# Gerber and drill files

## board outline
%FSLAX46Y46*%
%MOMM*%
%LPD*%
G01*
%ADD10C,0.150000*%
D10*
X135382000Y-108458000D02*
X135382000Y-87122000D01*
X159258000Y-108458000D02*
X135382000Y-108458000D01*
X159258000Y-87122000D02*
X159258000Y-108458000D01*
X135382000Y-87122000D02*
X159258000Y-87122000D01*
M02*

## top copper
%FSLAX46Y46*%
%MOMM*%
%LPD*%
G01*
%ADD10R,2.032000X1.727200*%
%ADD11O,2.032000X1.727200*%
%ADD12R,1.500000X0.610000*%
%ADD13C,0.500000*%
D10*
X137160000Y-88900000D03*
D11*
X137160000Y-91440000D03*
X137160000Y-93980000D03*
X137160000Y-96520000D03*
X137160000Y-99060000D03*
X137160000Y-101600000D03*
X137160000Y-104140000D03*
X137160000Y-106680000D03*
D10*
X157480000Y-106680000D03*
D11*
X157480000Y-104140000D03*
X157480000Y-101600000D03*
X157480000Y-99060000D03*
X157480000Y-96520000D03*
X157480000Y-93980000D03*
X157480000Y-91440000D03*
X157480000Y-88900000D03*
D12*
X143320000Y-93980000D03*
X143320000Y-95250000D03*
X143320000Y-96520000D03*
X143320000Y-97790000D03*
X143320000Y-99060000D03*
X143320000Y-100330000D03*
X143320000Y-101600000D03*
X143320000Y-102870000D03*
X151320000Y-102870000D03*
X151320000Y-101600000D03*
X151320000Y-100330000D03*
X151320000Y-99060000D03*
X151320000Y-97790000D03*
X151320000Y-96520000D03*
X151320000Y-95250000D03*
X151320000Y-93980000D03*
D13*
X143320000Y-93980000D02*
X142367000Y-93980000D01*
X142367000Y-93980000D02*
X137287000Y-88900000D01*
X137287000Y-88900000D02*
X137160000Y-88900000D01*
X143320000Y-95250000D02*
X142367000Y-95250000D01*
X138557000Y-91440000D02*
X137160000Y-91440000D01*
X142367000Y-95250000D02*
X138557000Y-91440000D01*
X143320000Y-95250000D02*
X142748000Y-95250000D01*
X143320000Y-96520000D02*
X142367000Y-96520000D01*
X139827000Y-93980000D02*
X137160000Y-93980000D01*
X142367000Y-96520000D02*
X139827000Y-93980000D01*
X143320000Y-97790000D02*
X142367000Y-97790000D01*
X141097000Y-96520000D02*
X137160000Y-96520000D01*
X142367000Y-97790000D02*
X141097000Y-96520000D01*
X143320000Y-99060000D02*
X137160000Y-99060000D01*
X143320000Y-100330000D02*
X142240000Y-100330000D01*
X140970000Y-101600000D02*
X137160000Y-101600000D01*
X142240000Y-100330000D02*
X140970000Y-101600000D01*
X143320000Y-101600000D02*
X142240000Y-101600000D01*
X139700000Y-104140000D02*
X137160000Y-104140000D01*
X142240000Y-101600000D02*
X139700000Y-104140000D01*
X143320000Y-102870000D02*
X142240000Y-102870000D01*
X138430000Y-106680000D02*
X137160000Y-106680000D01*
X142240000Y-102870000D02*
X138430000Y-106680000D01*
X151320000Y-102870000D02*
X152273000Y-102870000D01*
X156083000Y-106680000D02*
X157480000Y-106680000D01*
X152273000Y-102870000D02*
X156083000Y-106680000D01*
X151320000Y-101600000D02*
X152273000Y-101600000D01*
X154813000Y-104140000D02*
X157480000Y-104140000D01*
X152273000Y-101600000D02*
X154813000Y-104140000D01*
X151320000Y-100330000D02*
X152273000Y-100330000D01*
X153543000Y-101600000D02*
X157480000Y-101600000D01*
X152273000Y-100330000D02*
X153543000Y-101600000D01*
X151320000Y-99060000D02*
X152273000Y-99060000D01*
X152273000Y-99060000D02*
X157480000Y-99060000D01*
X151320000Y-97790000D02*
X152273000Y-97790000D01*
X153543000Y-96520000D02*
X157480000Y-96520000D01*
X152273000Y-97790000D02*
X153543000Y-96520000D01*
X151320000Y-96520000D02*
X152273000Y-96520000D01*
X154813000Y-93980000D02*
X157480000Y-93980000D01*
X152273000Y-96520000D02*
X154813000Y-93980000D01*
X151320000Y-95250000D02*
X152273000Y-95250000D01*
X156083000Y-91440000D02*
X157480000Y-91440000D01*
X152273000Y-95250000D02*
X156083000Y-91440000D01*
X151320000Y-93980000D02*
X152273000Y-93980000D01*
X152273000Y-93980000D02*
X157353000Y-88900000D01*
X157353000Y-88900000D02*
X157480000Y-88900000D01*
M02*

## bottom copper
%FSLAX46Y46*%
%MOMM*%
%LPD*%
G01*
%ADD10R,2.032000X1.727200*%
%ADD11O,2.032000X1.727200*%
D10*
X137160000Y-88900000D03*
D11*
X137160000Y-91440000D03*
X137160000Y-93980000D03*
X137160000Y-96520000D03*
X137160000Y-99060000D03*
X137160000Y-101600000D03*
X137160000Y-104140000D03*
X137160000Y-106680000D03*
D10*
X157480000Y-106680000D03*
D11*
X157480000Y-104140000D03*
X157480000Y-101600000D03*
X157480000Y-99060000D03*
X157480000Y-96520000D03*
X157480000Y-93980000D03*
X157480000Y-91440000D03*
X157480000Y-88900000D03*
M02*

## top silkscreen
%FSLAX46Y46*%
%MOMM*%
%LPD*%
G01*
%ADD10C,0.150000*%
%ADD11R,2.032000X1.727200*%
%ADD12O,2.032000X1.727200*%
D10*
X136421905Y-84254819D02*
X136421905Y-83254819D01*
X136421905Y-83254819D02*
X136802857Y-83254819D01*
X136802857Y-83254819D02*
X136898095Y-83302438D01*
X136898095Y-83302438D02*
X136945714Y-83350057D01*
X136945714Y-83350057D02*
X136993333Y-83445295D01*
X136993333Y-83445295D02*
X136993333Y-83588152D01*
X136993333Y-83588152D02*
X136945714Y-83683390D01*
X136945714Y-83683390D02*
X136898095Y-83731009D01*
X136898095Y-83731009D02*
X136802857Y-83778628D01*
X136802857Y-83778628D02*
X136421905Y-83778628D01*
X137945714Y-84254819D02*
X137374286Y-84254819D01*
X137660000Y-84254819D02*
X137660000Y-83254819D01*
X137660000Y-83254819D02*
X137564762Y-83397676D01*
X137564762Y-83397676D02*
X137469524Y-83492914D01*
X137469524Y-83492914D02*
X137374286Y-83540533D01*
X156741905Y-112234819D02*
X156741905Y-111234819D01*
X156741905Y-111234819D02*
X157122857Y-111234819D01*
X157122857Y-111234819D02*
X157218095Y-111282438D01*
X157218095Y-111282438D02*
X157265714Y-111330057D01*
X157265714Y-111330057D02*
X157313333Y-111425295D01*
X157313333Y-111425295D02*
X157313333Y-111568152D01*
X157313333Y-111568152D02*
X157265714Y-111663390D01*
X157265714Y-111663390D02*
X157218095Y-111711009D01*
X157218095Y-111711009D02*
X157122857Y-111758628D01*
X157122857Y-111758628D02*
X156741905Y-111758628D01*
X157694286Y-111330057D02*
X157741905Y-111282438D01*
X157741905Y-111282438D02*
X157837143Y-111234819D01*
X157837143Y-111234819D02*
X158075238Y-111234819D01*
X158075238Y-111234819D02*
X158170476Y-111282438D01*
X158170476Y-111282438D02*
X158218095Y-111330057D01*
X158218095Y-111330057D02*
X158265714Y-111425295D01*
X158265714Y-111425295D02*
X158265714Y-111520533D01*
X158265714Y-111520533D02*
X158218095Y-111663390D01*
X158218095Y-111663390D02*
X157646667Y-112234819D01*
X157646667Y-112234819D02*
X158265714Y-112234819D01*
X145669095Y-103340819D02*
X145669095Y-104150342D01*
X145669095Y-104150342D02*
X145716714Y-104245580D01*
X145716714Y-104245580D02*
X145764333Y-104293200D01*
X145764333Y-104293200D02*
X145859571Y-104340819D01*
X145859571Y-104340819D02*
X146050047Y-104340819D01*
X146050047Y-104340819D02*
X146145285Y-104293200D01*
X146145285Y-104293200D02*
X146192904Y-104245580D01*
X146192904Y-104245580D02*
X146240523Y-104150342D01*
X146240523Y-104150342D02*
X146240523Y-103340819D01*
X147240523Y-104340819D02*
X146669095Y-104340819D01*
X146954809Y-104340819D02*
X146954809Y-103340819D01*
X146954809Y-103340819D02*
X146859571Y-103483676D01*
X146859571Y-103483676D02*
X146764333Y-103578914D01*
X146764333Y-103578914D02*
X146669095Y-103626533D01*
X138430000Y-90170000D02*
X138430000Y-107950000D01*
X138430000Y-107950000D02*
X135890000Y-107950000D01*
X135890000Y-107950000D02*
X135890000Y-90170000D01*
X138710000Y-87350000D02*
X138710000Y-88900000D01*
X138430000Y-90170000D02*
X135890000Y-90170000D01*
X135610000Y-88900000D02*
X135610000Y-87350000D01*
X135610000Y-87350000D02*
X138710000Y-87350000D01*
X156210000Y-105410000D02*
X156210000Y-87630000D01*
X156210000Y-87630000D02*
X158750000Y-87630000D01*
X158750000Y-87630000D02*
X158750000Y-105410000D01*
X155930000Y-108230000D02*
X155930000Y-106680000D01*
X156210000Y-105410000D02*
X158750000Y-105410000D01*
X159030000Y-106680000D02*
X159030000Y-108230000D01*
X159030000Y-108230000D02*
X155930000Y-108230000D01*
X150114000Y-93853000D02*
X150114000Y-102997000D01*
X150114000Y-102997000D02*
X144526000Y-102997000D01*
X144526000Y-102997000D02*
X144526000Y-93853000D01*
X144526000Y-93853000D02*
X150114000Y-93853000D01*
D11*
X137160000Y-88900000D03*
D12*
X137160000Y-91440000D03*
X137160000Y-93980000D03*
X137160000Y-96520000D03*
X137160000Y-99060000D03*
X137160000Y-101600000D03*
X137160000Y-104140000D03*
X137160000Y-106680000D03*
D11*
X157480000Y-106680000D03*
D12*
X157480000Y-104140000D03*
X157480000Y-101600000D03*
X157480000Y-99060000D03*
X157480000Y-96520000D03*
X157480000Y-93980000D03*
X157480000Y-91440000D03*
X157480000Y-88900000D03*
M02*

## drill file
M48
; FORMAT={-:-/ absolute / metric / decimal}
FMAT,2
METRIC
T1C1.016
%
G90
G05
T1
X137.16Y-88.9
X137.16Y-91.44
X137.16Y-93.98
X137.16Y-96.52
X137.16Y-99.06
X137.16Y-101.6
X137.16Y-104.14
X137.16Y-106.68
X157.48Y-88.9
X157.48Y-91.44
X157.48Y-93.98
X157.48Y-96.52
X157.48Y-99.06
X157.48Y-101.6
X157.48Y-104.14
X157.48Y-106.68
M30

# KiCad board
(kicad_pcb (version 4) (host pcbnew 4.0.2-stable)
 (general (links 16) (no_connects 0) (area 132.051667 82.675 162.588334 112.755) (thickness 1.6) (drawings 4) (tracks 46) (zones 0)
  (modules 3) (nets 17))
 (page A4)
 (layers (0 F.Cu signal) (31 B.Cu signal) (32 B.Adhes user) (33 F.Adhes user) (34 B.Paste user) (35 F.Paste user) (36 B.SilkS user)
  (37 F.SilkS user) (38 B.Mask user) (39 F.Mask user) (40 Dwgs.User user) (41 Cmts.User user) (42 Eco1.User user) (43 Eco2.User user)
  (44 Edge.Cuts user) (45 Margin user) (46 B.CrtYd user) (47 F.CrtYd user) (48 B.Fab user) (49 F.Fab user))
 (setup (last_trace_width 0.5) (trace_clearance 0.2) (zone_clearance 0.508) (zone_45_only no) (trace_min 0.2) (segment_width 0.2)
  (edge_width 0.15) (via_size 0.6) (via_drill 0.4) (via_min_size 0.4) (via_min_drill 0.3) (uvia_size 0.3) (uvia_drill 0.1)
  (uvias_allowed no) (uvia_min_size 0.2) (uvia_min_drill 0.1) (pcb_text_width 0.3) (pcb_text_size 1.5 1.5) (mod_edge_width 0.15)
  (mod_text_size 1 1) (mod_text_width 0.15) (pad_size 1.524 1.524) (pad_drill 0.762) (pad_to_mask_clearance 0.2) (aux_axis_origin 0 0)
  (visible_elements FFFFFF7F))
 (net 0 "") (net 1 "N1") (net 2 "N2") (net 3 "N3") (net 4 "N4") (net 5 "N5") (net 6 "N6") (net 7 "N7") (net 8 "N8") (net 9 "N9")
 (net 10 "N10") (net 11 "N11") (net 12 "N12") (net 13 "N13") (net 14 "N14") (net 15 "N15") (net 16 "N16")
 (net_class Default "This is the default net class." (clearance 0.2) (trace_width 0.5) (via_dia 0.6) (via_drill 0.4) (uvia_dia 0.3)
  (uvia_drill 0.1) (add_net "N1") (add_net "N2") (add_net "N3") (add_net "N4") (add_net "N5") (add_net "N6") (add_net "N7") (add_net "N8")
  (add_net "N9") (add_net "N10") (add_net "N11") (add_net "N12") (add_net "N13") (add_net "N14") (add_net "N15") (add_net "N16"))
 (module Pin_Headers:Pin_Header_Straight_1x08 (layer F.Cu) (at 137.16 88.9)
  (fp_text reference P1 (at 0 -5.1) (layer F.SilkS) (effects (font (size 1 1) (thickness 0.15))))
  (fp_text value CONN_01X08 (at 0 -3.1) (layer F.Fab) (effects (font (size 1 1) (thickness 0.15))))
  (fp_line (start 1.27 1.27) (end 1.27 19.05) (layer F.SilkS) (width 0.15))
  (fp_line (start 1.27 19.05) (end -1.27 19.05) (layer F.SilkS) (width 0.15))
  (fp_line (start -1.27 19.05) (end -1.27 1.27) (layer F.SilkS) (width 0.15))
  (fp_line (start 1.55 -1.55) (end 1.55 0) (layer F.SilkS) (width 0.15))
  (fp_line (start 1.27 1.27) (end -1.27 1.27) (layer F.SilkS) (width 0.15))
  (fp_line (start -1.55 0) (end -1.55 -1.55) (layer F.SilkS) (width 0.15))
  (fp_line (start -1.55 -1.55) (end 1.55 -1.55) (layer F.SilkS) (width 0.15))
  (pad 1 thru_hole rect (at 0 0) (size 2.032 1.7272) (drill 1.016) (layers *.Cu *.Mask F.SilkS) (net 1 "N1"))
  (pad 2 thru_hole oval (at 0 2.54) (size 2.032 1.7272) (drill 1.016) (layers *.Cu *.Mask F.SilkS) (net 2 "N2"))
  (pad 3 thru_hole oval (at 0 5.08) (size 2.032 1.7272) (drill 1.016) (layers *.Cu *.Mask F.SilkS) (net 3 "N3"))
  (pad 4 thru_hole oval (at 0 7.62) (size 2.032 1.7272) (drill 1.016) (layers *.Cu *.Mask F.SilkS) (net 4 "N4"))
  (pad 5 thru_hole oval (at 0 10.16) (size 2.032 1.7272) (drill 1.016) (layers *.Cu *.Mask F.SilkS) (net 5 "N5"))
  (pad 6 thru_hole oval (at 0 12.7) (size 2.032 1.7272) (drill 1.016) (layers *.Cu *.Mask F.SilkS) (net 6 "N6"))
  (pad 7 thru_hole oval (at 0 15.24) (size 2.032 1.7272) (drill 1.016) (layers *.Cu *.Mask F.SilkS) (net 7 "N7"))
  (pad 8 thru_hole oval (at 0 17.78) (size 2.032 1.7272) (drill 1.016) (layers *.Cu *.Mask F.SilkS) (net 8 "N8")))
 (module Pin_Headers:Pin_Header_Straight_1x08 (layer F.Cu) (at 157.48 106.68 180)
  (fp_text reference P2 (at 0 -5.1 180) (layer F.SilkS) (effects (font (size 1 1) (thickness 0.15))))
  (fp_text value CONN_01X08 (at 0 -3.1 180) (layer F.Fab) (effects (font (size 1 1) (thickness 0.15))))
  (fp_line (start 1.27 1.27) (end 1.27 19.05) (layer F.SilkS) (width 0.15))
  (fp_line (start 1.27 19.05) (end -1.27 19.05) (layer F.SilkS) (width 0.15))
  (fp_line (start -1.27 19.05) (end -1.27 1.27) (layer F.SilkS) (width 0.15))
  (fp_line (start 1.55 -1.55) (end 1.55 0) (layer F.SilkS) (width 0.15))
  (fp_line (start 1.27 1.27) (end -1.27 1.27) (layer F.SilkS) (width 0.15))
  (fp_line (start -1.55 0) (end -1.55 -1.55) (layer F.SilkS) (width 0.15))
  (fp_line (start -1.55 -1.55) (end 1.55 -1.55) (layer F.SilkS) (width 0.15))
  (pad 1 thru_hole rect (at 0 0 180) (size 2.032 1.7272) (drill 1.016) (layers *.Cu *.Mask F.SilkS) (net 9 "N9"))
  (pad 2 thru_hole oval (at 0 2.54 180) (size 2.032 1.7272) (drill 1.016) (layers *.Cu *.Mask F.SilkS) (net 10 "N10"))
  (pad 3 thru_hole oval (at 0 5.08 180) (size 2.032 1.7272) (drill 1.016) (layers *.Cu *.Mask F.SilkS) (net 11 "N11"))
  (pad 4 thru_hole oval (at 0 7.62 180) (size 2.032 1.7272) (drill 1.016) (layers *.Cu *.Mask F.SilkS) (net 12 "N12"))
  (pad 5 thru_hole oval (at 0 10.16 180) (size 2.032 1.7272) (drill 1.016) (layers *.Cu *.Mask F.SilkS) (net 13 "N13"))
  (pad 6 thru_hole oval (at 0 12.7 180) (size 2.032 1.7272) (drill 1.016) (layers *.Cu *.Mask F.SilkS) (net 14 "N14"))
  (pad 7 thru_hole oval (at 0 15.24 180) (size 2.032 1.7272) (drill 1.016) (layers *.Cu *.Mask F.SilkS) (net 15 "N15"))
  (pad 8 thru_hole oval (at 0 17.78 180) (size 2.032 1.7272) (drill 1.016) (layers *.Cu *.Mask F.SilkS) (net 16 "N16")))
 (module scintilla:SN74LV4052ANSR (layer F.Cu) (at 147.32 99.06 270)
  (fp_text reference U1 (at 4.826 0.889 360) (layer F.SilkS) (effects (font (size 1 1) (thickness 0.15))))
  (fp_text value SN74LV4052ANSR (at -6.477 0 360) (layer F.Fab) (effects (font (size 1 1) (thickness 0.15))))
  (fp_line (start -5.207 -2.794) (end 3.937 -2.794) (layer F.SilkS) (width 0.15))
  (fp_line (start 3.937 -2.794) (end 3.937 2.794) (layer F.SilkS) (width 0.15))
  (fp_line (start 3.937 2.794) (end -5.207 2.794) (layer F.SilkS) (width 0.15))
  (fp_line (start -5.207 2.794) (end -5.207 -2.794) (layer F.SilkS) (width 0.15))
  (pad 1 smd rect (at -5.08 4 270) (size 0.61 1.5) (layers F.Cu F.Paste F.Mask) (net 1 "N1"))
  (pad 2 smd rect (at -3.81 4 270) (size 0.61 1.5) (layers F.Cu F.Paste F.Mask) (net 2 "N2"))
  (pad 3 smd rect (at -2.54 4 270) (size 0.61 1.5) (layers F.Cu F.Paste F.Mask) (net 3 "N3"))
  (pad 4 smd rect (at -1.27 4 270) (size 0.61 1.5) (layers F.Cu F.Paste F.Mask) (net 4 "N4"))
  (pad 5 smd rect (at 0 4 270) (size 0.61 1.5) (layers F.Cu F.Paste F.Mask) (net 5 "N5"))
  (pad 6 smd rect (at 1.27 4 270) (size 0.61 1.5) (layers F.Cu F.Paste F.Mask) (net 6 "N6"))
  (pad 7 smd rect (at 2.54 4 270) (size 0.61 1.5) (layers F.Cu F.Paste F.Mask) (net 7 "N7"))
  (pad 8 smd rect (at 3.81 4 270) (size 0.61 1.5) (layers F.Cu F.Paste F.Mask) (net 8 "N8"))
  (pad 9 smd rect (at 3.81 -4 270) (size 0.61 1.5) (layers F.Cu F.Paste F.Mask) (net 9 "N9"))
  (pad 10 smd rect (at 2.54 -4 270) (size 0.61 1.5) (layers F.Cu F.Paste F.Mask) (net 10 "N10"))
  (pad 11 smd rect (at 1.27 -4 270) (size 0.61 1.5) (layers F.Cu F.Paste F.Mask) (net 11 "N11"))
  (pad 12 smd rect (at 0 -4 270) (size 0.61 1.5) (layers F.Cu F.Paste F.Mask) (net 12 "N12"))
  (pad 13 smd rect (at -1.27 -4 270) (size 0.61 1.5) (layers F.Cu F.Paste F.Mask) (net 13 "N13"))
  (pad 14 smd rect (at -2.54 -4 270) (size 0.61 1.5) (layers F.Cu F.Paste F.Mask) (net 14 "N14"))
  (pad 15 smd rect (at -3.81 -4 270) (size 0.61 1.5) (layers F.Cu F.Paste F.Mask) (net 15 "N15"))
  (pad 16 smd rect (at -5.08 -4 270) (size 0.61 1.5) (layers F.Cu F.Paste F.Mask) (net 16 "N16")))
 (gr_line (start 135.382 108.458) (end 135.382 87.122) (angle 90) (layer Edge.Cuts) (width 0.15))
 (gr_line (start 159.258 108.458) (end 135.382 108.458) (angle 90) (layer Edge.Cuts) (width 0.15))
 (gr_line (start 159.258 87.122) (end 159.258 108.458) (angle 90) (layer Edge.Cuts) (width 0.15))
 (gr_line (start 135.382 87.122) (end 159.258 87.122) (angle 90) (layer Edge.Cuts) (width 0.15))
 (segment (start 143.32 93.98) (end 142.367 93.98) (width 0.5) (layer F.Cu) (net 1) (status 400000))
 (segment (start 142.367 93.98) (end 137.287 88.9) (width 0.5) (layer F.Cu) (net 1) (status 800000))
 (segment (start 137.287 88.9) (end 137.16 88.9) (width 0.5) (layer F.Cu) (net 1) (status C00000))
 (segment (start 143.32 95.25) (end 142.367 95.25) (width 0.5) (layer F.Cu) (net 2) (status 400000))
 (segment (start 138.557 91.44) (end 137.16 91.44) (width 0.5) (layer F.Cu) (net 2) (status 800000))
 (segment (start 142.367 95.25) (end 138.557 91.44) (width 0.5) (layer F.Cu) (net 2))
 (segment (start 143.32 95.25) (end 142.748 95.25) (width 0.5) (layer F.Cu) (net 2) (status C00000))
 (segment (start 143.32 96.52) (end 142.367 96.52) (width 0.5) (layer F.Cu) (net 3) (status 400000))
 (segment (start 139.827 93.98) (end 137.16 93.98) (width 0.5) (layer F.Cu) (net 3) (status 800000))
 (segment (start 142.367 96.52) (end 139.827 93.98) (width 0.5) (layer F.Cu) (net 3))
 (segment (start 143.32 97.79) (end 142.367 97.79) (width 0.5) (layer F.Cu) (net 4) (status 400000))
 (segment (start 141.097 96.52) (end 137.16 96.52) (width 0.5) (layer F.Cu) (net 4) (status 800000))
 (segment (start 142.367 97.79) (end 141.097 96.52) (width 0.5) (layer F.Cu) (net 4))
 (segment (start 143.32 99.06) (end 137.16 99.06) (width 0.5) (layer F.Cu) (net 5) (status C00000))
 (segment (start 143.32 100.33) (end 142.24 100.33) (width 0.5) (layer F.Cu) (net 6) (status 400000))
 (segment (start 140.97 101.6) (end 137.16 101.6) (width 0.5) (layer F.Cu) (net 6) (status 800000))
 (segment (start 142.24 100.33) (end 140.97 101.6) (width 0.5) (layer F.Cu) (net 6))
 (segment (start 143.32 101.6) (end 142.24 101.6) (width 0.5) (layer F.Cu) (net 7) (status 400000))
 (segment (start 139.7 104.14) (end 137.16 104.14) (width 0.5) (layer F.Cu) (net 7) (status 800000))
 (segment (start 142.24 101.6) (end 139.7 104.14) (width 0.5) (layer F.Cu) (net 7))
 (segment (start 143.32 102.87) (end 142.24 102.87) (width 0.5) (layer F.Cu) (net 8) (status 400000))
 (segment (start 138.43 106.68) (end 137.16 106.68) (width 0.5) (layer F.Cu) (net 8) (status 800000))
 (segment (start 142.24 102.87) (end 138.43 106.68) (width 0.5) (layer F.Cu) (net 8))
 (segment (start 151.32 102.87) (end 152.273 102.87) (width 0.5) (layer F.Cu) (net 9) (status 400000))
 (segment (start 156.083 106.68) (end 157.48 106.68) (width 0.5) (layer F.Cu) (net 9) (status 800000))
 (segment (start 152.273 102.87) (end 156.083 106.68) (width 0.5) (layer F.Cu) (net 9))
 (segment (start 151.32 101.6) (end 152.273 101.6) (width 0.5) (layer F.Cu) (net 10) (status 400000))
 (segment (start 154.813 104.14) (end 157.48 104.14) (width 0.5) (layer F.Cu) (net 10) (status 800000))
 (segment (start 152.273 101.6) (end 154.813 104.14) (width 0.5) (layer F.Cu) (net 10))
 (segment (start 151.32 100.33) (end 152.273 100.33) (width 0.5) (layer F.Cu) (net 11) (status 400000))
 (segment (start 153.543 101.6) (end 157.48 101.6) (width 0.5) (layer F.Cu) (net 11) (status 800000))
 (segment (start 152.273 100.33) (end 153.543 101.6) (width 0.5) (layer F.Cu) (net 11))
 (segment (start 151.32 99.06) (end 152.273 99.06) (width 0.5) (layer F.Cu) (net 12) (status 400000))
 (segment (start 152.273 99.06) (end 157.48 99.06) (width 0.5) (layer F.Cu) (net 12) (status 800000))
 (segment (start 151.32 97.79) (end 152.273 97.79) (width 0.5) (layer F.Cu) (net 13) (status 400000))
 (segment (start 153.543 96.52) (end 157.48 96.52) (width 0.5) (layer F.Cu) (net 13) (status 800000))
 (segment (start 152.273 97.79) (end 153.543 96.52) (width 0.5) (layer F.Cu) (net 13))
 (segment (start 151.32 96.52) (end 152.273 96.52) (width 0.5) (layer F.Cu) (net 14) (status 400000))
 (segment (start 154.813 93.98) (end 157.48 93.98) (width 0.5) (layer F.Cu) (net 14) (status 800000))
 (segment (start 152.273 96.52) (end 154.813 93.98) (width 0.5) (layer F.Cu) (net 14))
 (segment (start 151.32 95.25) (end 152.273 95.25) (width 0.5) (layer F.Cu) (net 15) (status 400000))
 (segment (start 156.083 91.44) (end 157.48 91.44) (width 0.5) (layer F.Cu) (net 15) (status 800000))
 (segment (start 152.273 95.25) (end 156.083 91.44) (width 0.5) (layer F.Cu) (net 15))
 (segment (start 151.32 93.98) (end 152.273 93.98) (width 0.5) (layer F.Cu) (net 16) (status 400000))
 (segment (start 152.273 93.98) (end 157.353 88.9) (width 0.5) (layer F.Cu) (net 16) (status 800000))
 (segment (start 157.353 88.9) (end 157.48 88.9) (width 0.5) (layer F.Cu) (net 16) (status C00000)))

